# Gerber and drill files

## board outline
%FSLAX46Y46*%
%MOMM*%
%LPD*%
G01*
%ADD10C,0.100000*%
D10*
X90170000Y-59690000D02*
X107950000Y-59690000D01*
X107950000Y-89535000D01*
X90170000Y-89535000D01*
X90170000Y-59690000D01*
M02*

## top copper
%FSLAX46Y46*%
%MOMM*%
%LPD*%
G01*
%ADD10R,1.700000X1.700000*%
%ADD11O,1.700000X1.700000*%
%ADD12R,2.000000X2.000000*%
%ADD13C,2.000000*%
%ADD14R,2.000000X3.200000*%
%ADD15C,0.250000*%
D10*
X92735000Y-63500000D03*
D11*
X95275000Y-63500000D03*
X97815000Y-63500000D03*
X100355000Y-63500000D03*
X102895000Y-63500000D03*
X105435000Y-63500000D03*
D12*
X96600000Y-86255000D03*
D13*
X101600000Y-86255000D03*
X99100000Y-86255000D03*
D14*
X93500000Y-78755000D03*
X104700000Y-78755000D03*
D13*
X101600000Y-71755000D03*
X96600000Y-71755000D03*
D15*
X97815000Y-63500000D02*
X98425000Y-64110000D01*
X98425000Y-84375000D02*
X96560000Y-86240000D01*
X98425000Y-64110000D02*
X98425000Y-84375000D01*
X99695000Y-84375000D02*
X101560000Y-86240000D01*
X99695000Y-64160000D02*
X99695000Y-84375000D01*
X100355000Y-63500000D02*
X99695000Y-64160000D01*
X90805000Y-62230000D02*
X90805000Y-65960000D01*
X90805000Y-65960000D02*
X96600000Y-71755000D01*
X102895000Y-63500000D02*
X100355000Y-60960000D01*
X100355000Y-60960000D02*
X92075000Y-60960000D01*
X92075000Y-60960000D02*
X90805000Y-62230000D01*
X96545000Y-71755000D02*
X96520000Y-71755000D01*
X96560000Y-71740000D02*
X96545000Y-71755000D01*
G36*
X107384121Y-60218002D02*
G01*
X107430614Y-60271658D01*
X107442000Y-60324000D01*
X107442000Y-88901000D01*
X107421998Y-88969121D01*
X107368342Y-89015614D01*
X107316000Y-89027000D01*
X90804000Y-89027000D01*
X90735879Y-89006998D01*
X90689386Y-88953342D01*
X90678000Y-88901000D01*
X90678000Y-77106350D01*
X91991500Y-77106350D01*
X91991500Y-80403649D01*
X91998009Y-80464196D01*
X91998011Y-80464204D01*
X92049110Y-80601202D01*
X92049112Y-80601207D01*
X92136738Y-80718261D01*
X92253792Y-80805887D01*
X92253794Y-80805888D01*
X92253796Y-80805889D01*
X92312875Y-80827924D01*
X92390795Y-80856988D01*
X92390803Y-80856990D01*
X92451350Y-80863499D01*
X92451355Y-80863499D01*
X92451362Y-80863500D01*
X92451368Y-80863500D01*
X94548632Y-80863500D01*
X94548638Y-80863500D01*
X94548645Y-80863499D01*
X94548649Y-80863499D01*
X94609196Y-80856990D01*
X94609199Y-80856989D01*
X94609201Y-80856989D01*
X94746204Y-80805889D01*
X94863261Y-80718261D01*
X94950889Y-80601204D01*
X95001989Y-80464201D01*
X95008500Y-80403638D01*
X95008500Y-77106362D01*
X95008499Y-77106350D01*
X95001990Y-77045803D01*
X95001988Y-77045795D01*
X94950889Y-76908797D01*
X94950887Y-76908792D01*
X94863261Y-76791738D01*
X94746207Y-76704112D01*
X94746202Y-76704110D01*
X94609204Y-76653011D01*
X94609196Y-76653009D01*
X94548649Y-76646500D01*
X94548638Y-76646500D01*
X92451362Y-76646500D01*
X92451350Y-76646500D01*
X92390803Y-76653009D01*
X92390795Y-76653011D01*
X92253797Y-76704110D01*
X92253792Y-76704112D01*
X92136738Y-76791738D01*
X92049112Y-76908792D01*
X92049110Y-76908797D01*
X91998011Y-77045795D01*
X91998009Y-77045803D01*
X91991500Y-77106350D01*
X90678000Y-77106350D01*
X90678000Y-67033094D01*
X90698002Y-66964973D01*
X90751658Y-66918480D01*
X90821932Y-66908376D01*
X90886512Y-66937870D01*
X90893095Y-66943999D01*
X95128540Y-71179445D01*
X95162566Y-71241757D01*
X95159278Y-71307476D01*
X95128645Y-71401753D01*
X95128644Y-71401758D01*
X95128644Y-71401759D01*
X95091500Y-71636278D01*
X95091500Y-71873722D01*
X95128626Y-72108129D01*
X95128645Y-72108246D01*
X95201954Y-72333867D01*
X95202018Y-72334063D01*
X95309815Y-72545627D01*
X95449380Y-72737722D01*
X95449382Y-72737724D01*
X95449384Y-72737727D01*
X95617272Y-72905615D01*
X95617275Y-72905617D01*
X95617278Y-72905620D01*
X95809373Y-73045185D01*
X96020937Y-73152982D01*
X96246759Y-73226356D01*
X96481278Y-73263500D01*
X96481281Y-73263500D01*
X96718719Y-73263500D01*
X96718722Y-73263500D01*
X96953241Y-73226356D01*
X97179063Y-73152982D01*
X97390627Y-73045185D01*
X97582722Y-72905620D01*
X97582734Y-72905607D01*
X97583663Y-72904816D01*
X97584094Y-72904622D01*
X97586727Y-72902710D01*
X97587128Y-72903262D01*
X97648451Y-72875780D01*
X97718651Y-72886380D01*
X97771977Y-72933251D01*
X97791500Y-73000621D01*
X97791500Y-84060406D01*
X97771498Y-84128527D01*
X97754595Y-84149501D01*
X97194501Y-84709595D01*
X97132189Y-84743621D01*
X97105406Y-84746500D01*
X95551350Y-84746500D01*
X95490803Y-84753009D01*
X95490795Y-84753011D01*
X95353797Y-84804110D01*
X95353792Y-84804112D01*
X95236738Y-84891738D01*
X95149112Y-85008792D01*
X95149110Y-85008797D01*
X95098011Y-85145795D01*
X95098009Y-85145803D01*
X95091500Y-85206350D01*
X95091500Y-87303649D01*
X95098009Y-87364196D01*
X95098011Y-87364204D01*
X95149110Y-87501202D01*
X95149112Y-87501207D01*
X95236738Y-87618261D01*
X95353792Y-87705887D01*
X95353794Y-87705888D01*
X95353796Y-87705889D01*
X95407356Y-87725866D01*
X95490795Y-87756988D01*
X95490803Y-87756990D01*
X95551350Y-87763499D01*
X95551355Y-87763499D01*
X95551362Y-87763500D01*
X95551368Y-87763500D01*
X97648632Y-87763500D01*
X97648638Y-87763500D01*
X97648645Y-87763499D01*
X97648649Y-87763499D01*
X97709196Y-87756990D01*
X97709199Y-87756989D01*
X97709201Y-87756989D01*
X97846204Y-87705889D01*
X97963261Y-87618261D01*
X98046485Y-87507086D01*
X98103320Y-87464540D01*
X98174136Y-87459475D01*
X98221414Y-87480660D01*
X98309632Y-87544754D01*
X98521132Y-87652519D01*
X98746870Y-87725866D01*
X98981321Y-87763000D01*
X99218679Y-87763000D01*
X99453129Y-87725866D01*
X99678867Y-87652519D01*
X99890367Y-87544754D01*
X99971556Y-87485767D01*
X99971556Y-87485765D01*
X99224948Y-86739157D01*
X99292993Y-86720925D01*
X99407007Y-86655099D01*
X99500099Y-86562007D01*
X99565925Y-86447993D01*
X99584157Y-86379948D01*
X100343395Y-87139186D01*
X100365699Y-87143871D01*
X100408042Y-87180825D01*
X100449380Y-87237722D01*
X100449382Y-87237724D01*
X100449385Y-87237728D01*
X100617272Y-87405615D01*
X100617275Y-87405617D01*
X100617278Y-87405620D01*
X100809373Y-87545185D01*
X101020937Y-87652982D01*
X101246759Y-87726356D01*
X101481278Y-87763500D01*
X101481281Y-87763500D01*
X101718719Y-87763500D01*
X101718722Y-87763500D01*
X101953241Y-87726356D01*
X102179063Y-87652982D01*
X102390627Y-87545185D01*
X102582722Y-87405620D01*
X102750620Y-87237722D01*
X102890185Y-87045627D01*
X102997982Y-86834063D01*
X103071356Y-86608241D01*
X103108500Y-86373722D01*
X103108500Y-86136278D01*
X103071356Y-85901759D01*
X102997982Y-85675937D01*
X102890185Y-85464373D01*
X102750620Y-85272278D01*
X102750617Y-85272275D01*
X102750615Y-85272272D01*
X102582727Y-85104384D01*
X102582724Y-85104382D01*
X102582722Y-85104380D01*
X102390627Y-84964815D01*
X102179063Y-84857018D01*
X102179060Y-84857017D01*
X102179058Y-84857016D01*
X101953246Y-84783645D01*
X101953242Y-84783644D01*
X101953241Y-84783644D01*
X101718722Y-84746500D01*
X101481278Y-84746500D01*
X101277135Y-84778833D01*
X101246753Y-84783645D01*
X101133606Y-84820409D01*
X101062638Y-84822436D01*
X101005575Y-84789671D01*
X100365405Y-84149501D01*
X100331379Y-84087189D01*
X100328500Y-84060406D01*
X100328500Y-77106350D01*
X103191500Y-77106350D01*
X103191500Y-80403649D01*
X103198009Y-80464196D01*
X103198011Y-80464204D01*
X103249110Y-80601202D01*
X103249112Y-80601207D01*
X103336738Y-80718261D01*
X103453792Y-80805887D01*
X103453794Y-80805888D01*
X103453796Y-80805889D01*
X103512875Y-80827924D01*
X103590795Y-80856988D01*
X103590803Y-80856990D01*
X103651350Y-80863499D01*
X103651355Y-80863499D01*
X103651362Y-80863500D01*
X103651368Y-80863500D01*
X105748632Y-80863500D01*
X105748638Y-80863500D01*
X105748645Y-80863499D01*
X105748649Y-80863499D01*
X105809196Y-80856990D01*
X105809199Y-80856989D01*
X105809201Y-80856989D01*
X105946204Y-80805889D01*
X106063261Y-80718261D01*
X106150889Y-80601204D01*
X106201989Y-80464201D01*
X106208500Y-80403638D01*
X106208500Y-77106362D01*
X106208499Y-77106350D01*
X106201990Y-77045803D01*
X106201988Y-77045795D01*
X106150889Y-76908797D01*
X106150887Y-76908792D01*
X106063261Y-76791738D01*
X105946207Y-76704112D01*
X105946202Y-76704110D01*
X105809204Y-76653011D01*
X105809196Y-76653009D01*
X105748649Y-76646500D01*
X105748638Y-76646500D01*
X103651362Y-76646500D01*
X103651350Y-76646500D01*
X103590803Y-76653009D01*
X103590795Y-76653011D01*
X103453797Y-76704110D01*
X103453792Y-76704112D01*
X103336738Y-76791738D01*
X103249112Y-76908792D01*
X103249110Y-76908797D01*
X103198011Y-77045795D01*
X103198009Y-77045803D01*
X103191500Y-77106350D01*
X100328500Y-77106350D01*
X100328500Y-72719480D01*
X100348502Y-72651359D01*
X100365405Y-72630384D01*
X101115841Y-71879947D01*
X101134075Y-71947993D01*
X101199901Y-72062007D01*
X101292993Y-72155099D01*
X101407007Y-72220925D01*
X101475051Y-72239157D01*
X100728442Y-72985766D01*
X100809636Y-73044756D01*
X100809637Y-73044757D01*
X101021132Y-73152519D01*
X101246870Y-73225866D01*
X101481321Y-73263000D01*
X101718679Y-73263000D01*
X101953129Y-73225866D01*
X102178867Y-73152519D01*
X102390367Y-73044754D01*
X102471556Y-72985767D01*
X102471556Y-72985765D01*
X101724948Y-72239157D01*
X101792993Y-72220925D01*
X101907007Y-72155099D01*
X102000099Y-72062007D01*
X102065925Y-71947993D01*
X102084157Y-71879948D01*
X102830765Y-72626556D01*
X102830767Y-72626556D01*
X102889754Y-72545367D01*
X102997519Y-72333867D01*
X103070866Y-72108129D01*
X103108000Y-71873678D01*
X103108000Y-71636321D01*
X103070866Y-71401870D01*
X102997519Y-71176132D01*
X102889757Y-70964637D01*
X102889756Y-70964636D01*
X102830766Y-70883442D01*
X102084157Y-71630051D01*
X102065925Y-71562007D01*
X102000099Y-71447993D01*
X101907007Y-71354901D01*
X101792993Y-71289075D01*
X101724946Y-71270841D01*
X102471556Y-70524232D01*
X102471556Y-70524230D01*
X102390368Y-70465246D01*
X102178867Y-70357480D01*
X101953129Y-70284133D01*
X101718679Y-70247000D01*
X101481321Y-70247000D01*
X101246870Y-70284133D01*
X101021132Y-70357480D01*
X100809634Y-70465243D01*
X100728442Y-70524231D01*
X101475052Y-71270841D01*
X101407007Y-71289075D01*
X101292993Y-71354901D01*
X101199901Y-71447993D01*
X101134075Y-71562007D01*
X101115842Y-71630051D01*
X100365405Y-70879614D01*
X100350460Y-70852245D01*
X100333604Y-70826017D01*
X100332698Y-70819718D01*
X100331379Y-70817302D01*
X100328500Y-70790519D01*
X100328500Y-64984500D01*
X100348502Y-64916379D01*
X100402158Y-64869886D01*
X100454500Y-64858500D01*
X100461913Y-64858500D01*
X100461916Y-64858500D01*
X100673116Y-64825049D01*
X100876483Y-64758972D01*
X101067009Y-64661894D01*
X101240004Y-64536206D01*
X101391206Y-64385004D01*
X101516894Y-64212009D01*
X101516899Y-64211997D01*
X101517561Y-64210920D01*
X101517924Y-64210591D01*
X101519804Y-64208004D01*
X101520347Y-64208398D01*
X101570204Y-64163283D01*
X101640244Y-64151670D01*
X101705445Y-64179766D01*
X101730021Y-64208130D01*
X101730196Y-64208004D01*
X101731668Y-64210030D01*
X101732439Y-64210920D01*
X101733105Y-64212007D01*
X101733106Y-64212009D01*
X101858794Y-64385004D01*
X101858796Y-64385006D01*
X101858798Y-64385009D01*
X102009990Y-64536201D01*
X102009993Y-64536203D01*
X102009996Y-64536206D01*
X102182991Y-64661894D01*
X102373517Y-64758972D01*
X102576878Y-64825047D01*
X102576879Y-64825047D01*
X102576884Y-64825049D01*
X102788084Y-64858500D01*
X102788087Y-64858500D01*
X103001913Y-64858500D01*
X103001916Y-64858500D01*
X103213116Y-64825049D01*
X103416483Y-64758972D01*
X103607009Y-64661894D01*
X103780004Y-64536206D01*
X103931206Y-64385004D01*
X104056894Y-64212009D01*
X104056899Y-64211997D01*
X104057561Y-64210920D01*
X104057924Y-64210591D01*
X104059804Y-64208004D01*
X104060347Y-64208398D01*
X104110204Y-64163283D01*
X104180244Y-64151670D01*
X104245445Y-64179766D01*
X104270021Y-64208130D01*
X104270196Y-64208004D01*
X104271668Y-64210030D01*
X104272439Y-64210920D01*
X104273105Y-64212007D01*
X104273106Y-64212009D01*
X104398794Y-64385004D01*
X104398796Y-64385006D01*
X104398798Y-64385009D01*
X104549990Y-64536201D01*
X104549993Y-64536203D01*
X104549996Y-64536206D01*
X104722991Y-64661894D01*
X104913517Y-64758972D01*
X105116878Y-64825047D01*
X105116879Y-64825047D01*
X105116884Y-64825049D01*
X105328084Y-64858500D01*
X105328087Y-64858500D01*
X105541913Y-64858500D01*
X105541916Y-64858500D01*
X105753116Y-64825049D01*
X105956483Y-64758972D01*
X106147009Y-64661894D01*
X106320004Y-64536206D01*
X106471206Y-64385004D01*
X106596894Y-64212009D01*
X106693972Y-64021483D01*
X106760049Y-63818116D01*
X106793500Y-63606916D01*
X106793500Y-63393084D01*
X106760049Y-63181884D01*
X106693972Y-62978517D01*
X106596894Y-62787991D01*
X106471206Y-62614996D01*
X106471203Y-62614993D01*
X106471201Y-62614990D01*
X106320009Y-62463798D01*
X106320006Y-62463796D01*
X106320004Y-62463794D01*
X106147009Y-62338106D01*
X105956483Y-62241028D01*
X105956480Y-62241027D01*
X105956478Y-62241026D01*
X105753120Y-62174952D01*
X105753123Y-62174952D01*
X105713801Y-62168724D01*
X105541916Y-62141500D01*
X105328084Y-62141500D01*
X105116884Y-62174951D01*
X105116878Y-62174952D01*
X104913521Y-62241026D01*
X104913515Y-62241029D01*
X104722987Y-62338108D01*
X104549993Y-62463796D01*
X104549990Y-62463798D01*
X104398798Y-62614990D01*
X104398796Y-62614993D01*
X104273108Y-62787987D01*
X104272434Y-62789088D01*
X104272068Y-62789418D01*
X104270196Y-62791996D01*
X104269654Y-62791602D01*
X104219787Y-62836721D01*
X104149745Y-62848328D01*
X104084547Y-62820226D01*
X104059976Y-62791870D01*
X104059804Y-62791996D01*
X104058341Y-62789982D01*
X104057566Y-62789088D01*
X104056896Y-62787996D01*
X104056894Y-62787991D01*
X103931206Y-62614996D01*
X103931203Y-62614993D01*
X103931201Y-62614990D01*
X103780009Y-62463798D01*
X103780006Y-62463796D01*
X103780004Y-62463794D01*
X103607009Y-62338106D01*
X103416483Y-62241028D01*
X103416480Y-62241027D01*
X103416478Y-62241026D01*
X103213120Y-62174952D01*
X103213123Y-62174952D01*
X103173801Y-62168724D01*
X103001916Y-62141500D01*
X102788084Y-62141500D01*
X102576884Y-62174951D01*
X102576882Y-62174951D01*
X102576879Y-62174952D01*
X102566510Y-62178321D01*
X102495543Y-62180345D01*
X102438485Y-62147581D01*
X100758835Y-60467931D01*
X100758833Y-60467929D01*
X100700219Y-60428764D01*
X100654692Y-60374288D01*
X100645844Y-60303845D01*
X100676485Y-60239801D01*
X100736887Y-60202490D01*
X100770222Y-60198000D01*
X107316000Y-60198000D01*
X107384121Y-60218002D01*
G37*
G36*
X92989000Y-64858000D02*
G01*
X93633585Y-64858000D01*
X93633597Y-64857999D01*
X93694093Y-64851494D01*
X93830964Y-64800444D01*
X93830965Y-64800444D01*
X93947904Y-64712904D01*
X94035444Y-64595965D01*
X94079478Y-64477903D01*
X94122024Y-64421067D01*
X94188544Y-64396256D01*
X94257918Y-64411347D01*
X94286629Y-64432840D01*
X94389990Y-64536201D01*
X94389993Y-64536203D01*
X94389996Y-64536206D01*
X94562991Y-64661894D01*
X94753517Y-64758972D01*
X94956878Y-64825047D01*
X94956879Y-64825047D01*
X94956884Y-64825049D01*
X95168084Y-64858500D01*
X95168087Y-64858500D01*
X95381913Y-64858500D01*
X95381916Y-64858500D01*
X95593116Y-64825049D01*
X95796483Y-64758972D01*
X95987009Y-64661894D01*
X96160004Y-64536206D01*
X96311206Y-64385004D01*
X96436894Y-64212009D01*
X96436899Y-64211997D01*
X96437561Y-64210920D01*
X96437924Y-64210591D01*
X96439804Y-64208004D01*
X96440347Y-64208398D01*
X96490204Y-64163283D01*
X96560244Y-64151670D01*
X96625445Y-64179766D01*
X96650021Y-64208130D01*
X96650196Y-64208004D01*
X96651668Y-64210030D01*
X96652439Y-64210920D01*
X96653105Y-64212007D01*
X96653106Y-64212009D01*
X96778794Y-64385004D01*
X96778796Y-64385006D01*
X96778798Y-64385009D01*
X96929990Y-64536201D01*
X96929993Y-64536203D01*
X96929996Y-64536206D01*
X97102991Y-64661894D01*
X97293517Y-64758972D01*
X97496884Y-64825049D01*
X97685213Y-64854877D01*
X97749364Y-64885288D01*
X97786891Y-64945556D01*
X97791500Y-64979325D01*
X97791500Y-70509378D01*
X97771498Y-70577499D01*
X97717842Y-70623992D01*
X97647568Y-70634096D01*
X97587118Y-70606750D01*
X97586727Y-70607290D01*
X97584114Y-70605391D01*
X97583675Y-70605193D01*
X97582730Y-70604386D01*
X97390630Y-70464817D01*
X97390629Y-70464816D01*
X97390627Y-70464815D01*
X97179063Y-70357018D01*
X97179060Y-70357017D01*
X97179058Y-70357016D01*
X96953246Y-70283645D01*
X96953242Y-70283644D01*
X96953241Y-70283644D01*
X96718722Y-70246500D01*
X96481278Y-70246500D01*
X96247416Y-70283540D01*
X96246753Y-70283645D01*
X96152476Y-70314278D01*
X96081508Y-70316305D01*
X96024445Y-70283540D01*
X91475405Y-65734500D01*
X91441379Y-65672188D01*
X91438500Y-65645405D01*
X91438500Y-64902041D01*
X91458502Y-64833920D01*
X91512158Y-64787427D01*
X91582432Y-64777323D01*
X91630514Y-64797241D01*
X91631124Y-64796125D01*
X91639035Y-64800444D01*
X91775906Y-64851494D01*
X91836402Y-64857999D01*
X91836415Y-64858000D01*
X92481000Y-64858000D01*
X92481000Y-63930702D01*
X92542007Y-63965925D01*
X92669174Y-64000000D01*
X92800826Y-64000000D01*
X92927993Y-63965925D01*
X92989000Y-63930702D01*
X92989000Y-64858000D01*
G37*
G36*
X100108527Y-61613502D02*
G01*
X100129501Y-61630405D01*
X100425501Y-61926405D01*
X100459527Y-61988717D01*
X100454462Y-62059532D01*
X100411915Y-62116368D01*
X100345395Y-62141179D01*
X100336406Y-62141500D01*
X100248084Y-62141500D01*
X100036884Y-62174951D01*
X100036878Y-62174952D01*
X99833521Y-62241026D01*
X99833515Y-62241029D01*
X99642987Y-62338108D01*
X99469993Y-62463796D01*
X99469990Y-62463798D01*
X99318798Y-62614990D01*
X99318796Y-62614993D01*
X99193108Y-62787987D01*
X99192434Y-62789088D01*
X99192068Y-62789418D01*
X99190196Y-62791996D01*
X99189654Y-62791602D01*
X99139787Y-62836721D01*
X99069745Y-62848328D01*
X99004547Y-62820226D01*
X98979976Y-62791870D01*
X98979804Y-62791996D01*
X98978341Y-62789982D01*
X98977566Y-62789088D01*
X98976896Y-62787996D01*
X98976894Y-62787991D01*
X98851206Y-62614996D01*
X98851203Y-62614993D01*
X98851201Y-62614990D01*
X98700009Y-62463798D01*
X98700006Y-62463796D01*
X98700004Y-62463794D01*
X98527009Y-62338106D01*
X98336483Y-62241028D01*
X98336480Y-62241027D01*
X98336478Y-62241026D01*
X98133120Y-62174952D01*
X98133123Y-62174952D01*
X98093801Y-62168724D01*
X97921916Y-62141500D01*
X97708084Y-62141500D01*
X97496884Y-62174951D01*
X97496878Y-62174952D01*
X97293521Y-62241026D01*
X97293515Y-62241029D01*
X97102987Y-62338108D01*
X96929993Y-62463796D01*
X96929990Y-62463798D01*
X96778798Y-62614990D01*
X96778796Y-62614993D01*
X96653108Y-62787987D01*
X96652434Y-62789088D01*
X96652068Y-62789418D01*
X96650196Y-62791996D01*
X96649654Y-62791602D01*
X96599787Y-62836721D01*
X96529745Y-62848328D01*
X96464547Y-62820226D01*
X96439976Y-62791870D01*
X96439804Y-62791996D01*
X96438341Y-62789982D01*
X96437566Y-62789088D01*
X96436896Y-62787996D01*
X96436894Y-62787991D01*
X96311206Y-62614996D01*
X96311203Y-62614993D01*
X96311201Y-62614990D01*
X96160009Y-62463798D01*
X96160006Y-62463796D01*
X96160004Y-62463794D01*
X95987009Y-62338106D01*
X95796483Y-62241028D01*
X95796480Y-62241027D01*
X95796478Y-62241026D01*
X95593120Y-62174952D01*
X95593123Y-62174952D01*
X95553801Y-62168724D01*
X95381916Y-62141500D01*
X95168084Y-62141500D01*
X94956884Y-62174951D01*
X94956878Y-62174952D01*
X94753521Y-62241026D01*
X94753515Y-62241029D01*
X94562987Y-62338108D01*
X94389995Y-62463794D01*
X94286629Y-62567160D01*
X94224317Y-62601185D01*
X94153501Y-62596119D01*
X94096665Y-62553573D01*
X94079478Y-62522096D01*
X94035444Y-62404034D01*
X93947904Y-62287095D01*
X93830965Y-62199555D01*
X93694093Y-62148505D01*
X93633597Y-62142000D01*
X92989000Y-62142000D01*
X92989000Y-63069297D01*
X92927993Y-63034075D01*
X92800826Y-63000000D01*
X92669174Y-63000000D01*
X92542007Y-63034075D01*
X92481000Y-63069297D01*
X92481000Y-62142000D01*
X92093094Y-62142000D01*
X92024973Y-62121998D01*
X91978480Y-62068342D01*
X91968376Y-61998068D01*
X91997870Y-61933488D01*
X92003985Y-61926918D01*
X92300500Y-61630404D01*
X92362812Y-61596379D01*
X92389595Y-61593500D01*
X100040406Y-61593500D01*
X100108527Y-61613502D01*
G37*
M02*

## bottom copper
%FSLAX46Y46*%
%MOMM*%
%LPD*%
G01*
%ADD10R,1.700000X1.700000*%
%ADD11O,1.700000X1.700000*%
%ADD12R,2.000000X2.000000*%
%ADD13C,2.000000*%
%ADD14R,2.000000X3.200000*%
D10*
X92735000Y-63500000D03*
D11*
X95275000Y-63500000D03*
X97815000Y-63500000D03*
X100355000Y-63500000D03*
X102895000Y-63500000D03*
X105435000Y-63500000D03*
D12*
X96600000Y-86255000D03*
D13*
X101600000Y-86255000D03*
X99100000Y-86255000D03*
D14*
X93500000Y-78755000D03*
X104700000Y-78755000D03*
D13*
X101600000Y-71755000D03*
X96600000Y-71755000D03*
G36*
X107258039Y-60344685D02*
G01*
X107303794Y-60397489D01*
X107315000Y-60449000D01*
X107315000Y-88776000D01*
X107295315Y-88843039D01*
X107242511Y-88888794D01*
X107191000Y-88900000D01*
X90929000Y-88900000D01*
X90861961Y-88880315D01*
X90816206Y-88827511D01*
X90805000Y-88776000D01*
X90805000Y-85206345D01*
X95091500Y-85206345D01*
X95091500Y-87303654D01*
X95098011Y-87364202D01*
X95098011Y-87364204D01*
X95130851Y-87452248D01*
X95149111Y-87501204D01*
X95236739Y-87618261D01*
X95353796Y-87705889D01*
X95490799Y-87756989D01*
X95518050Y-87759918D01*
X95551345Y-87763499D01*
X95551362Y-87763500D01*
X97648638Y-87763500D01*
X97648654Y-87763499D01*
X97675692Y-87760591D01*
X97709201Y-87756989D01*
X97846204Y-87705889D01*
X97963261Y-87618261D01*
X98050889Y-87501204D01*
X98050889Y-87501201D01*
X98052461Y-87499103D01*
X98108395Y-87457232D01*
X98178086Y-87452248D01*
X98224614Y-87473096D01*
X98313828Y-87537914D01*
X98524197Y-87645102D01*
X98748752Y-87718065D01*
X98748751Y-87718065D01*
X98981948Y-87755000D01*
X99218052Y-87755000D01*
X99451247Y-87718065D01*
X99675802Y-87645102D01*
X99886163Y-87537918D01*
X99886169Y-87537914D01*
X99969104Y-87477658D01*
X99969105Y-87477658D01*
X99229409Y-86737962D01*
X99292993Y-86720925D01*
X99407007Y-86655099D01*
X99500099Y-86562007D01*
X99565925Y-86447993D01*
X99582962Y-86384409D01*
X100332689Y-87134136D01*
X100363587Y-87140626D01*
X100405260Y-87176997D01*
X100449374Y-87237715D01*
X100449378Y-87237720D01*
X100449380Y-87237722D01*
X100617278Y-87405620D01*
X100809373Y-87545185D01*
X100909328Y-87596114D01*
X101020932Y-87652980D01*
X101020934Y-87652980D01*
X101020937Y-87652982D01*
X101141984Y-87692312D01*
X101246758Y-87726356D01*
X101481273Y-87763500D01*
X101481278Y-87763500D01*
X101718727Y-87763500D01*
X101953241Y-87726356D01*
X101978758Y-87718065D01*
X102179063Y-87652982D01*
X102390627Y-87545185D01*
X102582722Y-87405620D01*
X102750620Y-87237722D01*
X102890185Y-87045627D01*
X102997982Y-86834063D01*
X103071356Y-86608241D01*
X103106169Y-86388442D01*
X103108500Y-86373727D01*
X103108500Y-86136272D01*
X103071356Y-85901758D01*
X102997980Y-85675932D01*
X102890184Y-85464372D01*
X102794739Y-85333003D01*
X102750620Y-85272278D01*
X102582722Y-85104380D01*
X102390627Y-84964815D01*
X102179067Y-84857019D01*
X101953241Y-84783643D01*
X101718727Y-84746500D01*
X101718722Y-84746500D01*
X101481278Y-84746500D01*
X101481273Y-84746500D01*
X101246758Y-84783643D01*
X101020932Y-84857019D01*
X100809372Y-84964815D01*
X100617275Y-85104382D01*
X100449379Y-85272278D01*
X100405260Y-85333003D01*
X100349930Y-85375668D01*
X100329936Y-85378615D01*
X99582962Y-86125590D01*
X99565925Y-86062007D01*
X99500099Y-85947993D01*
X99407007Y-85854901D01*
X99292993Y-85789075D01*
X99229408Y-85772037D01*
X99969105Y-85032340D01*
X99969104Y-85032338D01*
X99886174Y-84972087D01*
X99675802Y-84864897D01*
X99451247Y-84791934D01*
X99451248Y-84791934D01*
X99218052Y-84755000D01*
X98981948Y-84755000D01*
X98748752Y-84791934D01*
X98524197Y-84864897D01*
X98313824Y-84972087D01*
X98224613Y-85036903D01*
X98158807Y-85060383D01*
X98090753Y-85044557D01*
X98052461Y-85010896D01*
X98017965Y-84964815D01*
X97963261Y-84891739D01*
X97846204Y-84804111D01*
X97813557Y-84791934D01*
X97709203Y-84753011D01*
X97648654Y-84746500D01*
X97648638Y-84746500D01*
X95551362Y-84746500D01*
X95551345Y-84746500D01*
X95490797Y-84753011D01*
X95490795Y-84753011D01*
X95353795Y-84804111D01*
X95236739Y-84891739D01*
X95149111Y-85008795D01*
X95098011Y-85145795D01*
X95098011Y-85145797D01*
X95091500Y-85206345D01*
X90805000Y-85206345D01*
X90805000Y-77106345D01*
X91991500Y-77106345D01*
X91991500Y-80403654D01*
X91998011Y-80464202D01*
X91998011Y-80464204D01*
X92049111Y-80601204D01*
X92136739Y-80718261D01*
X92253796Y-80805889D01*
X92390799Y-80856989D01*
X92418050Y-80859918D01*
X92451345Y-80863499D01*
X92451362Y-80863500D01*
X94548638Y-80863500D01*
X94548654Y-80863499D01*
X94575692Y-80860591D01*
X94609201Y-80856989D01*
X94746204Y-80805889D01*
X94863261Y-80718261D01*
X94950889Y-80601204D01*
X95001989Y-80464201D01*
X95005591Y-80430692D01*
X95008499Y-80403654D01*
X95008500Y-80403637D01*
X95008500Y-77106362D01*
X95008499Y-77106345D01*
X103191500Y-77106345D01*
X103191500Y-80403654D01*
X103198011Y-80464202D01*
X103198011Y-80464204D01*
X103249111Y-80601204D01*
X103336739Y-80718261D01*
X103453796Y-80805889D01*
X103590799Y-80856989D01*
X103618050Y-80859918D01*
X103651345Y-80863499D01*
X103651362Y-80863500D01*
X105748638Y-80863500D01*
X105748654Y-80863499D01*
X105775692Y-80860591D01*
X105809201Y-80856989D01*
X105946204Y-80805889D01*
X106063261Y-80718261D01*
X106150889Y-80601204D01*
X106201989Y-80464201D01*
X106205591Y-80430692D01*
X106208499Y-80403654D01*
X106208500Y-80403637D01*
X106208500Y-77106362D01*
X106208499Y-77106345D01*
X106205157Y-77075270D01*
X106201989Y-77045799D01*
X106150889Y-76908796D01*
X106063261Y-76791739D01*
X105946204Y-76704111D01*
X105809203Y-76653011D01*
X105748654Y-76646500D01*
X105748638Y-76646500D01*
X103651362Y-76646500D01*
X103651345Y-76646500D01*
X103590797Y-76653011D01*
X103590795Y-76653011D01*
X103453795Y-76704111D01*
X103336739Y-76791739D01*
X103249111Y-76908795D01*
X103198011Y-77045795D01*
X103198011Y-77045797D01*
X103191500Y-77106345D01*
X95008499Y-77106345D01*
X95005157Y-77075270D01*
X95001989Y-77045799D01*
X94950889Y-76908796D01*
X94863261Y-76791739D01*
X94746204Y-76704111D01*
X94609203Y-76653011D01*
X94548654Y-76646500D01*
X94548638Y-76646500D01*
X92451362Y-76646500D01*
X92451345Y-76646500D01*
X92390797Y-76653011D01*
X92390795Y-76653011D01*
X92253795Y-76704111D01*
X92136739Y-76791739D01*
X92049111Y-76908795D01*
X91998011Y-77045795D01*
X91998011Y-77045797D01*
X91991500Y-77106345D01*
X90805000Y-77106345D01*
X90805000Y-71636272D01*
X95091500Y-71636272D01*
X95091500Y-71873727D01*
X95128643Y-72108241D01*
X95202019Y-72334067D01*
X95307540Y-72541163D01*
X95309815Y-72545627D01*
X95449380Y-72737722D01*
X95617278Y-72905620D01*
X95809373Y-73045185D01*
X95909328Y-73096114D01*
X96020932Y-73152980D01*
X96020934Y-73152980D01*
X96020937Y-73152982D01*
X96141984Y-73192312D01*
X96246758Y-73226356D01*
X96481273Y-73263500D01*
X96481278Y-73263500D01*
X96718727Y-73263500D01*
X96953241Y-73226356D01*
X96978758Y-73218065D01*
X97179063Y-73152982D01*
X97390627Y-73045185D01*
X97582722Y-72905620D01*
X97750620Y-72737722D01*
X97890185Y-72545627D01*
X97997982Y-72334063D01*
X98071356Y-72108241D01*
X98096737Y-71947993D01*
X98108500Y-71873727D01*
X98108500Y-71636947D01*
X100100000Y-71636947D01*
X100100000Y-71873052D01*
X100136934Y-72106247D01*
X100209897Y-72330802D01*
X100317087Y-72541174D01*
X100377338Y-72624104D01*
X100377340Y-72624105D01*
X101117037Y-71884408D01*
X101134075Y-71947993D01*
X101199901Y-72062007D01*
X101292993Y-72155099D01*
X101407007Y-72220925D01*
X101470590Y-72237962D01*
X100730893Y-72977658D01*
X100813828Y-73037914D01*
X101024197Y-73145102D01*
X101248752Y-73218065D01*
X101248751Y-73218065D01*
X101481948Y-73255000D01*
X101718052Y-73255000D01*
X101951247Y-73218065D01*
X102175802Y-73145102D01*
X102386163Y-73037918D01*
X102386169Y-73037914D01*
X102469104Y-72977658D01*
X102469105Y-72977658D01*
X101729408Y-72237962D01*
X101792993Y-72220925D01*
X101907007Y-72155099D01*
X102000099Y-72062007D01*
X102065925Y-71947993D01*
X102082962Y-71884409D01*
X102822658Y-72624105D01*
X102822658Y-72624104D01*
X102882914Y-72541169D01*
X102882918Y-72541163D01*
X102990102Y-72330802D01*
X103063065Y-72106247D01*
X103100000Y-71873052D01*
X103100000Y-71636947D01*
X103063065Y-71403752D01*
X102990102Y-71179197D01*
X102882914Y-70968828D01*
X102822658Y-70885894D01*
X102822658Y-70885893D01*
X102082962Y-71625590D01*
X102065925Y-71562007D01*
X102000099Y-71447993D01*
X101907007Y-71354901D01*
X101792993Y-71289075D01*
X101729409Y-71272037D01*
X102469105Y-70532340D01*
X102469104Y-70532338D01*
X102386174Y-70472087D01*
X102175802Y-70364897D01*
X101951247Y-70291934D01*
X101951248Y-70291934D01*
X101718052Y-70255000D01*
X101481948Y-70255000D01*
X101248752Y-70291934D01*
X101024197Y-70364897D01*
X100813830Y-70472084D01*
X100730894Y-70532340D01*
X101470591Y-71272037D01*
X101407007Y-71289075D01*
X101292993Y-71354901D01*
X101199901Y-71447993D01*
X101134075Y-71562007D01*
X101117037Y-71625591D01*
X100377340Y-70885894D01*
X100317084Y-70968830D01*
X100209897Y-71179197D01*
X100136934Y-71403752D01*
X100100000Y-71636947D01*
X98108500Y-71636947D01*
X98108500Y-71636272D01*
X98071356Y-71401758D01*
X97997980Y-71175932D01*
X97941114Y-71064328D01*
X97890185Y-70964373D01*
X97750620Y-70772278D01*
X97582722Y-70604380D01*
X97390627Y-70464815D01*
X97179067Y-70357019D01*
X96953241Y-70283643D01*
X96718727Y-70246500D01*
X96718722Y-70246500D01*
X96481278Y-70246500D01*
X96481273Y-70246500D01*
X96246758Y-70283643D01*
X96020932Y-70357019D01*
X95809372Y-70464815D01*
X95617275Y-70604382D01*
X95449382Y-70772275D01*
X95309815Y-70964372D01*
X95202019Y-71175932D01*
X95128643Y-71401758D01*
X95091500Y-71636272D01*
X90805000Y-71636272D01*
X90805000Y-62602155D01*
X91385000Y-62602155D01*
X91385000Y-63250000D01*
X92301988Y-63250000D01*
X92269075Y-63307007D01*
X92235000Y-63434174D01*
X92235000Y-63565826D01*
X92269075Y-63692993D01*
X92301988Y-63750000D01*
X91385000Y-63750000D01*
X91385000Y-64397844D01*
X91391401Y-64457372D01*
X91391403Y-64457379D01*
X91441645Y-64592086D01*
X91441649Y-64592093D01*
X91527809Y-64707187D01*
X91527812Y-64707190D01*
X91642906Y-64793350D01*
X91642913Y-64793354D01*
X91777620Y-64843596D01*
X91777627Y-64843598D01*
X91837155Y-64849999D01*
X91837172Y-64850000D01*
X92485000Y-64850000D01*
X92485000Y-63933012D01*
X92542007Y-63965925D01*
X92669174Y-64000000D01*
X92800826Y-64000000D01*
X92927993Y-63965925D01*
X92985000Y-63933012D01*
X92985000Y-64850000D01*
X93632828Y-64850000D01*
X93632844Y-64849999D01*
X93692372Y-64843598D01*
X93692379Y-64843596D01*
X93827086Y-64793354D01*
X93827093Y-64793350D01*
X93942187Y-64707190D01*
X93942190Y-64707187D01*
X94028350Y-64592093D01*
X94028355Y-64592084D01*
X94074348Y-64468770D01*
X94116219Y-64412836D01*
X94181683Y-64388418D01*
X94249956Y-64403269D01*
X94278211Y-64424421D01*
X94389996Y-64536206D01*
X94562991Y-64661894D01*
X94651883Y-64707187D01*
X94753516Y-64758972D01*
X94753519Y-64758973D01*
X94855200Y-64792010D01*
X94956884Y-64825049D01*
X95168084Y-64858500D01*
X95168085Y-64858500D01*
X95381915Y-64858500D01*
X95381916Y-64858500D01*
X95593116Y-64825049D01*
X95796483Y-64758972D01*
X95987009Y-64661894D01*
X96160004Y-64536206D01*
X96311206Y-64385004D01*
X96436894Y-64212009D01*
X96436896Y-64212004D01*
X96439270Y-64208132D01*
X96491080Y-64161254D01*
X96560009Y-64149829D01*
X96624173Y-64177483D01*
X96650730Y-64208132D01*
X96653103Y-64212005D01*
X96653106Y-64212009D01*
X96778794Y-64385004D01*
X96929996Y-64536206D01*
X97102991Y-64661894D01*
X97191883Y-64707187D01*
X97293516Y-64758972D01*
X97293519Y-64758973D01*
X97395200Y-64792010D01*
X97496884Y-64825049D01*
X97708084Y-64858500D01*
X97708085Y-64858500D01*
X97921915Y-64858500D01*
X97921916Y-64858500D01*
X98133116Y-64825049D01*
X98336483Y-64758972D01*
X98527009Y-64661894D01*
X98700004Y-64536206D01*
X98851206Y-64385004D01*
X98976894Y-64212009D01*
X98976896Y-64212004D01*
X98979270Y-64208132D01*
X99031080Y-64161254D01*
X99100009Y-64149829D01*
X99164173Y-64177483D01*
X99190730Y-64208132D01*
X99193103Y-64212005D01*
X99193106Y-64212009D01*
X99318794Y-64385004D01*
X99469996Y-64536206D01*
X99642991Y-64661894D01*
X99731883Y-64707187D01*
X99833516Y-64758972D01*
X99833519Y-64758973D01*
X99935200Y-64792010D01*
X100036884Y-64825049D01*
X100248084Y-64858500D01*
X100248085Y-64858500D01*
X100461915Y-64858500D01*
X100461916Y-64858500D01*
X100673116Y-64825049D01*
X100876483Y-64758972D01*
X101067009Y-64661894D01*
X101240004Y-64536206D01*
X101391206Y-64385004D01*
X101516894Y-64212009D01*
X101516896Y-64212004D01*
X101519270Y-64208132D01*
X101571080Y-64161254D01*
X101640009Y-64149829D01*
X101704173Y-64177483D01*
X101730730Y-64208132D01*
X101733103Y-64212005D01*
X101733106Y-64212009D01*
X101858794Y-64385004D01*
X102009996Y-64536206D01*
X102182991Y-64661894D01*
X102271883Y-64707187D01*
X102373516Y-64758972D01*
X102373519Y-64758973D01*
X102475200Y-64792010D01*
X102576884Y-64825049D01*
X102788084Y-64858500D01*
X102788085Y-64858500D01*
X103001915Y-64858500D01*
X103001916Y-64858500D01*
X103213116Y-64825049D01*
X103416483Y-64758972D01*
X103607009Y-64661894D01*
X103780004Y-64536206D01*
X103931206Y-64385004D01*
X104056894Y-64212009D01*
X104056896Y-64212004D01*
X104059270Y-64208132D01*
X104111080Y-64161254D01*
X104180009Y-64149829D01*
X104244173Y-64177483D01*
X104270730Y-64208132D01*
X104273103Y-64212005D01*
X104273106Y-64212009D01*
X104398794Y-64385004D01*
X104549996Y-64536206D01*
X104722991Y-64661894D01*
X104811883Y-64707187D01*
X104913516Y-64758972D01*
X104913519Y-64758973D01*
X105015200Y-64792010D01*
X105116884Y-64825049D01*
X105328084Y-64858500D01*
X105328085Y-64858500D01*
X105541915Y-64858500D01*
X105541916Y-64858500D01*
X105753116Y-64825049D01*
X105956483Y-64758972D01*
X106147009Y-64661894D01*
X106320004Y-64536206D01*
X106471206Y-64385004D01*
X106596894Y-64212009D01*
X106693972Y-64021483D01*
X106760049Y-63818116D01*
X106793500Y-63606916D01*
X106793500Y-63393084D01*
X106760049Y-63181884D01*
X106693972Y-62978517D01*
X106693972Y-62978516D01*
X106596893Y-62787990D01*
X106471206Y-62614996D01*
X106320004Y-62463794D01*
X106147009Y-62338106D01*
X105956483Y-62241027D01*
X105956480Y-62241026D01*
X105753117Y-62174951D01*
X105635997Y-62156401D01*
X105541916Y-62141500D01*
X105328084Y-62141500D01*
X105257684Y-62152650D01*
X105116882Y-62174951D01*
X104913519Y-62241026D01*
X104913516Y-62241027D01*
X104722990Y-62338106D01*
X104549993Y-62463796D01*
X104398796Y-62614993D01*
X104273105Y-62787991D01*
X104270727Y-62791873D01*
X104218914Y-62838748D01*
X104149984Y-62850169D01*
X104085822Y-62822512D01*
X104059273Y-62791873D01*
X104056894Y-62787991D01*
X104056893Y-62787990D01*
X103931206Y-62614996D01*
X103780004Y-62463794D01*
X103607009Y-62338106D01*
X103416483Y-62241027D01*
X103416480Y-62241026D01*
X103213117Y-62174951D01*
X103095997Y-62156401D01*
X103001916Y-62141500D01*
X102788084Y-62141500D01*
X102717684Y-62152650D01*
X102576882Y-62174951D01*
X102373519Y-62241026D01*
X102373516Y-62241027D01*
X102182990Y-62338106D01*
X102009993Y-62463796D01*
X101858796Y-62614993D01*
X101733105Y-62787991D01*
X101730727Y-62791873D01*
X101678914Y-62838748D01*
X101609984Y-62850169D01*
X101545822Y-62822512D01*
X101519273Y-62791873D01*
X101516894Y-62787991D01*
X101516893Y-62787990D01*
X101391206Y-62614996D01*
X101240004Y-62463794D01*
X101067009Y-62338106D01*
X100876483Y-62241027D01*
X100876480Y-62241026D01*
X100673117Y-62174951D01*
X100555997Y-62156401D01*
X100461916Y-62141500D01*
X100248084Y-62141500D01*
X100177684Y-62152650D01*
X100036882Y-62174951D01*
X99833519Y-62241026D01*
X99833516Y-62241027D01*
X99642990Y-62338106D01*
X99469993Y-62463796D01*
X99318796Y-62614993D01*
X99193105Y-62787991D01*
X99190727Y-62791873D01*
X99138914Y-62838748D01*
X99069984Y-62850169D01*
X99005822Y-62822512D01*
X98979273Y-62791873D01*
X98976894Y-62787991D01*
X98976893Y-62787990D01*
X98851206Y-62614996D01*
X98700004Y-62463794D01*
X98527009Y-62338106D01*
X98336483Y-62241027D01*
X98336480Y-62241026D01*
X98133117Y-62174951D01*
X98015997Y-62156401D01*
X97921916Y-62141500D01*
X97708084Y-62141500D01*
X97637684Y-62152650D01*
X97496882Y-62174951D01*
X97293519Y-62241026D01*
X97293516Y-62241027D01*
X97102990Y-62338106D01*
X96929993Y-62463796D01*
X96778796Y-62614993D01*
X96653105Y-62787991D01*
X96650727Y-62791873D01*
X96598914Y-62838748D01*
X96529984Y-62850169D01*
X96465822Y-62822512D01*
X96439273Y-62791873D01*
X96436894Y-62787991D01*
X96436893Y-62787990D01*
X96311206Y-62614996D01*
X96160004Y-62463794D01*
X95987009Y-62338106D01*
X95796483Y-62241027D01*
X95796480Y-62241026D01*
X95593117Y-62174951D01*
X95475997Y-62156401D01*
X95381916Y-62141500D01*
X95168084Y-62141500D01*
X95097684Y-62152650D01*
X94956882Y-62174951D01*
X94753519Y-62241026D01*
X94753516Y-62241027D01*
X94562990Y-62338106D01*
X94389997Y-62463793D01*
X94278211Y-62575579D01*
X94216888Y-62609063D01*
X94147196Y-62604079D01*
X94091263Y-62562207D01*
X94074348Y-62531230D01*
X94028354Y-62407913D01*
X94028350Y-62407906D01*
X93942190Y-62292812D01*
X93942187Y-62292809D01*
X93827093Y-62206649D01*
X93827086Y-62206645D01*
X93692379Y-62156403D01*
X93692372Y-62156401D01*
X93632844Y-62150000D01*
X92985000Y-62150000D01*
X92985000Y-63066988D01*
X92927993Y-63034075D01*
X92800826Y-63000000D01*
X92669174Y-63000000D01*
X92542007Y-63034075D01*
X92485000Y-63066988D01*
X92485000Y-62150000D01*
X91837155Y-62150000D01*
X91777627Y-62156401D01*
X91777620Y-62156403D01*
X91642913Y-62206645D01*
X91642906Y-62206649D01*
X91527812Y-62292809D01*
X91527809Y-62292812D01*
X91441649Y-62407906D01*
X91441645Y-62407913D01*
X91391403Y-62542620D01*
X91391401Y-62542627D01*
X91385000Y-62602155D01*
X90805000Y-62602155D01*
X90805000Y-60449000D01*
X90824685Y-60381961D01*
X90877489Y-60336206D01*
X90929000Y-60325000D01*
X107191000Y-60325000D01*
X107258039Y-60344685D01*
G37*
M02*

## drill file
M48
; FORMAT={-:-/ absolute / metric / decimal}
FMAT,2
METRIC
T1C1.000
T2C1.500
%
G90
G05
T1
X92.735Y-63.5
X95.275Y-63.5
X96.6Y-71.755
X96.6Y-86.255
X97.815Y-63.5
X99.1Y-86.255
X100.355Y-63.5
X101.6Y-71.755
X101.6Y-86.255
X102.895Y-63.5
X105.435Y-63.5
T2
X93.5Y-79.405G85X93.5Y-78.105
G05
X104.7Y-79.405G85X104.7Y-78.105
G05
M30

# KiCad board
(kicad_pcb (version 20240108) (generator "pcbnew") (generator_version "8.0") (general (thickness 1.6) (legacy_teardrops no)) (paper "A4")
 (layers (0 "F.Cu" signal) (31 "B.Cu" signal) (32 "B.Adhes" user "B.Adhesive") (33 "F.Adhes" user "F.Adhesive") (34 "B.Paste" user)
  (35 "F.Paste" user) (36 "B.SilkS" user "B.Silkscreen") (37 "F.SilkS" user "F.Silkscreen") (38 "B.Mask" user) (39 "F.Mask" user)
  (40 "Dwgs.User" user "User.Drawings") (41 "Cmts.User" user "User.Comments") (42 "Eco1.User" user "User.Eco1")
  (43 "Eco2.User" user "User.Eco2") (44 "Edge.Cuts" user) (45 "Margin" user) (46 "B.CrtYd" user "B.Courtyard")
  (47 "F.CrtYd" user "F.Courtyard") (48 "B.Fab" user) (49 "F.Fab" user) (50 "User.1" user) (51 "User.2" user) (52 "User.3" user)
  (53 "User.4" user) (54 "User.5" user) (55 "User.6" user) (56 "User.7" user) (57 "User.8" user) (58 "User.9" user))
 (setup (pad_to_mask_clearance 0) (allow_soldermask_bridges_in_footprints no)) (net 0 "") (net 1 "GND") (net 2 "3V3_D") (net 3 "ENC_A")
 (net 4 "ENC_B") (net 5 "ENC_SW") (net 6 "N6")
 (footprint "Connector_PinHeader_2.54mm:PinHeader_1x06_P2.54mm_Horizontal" (layer "F.Cu") (at 92.735 63.5 90)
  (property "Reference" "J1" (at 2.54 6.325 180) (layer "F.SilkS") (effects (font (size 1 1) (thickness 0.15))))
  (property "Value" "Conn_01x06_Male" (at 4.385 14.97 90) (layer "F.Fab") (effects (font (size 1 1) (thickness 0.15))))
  (pad "1" thru_hole rect (at 0 0 90) (size 1.7 1.7) (drill 1) (layers "*.Cu" "*.Mask") (remove_unused_layers no) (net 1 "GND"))
  (pad "2" thru_hole oval (at 0 2.54 90) (size 1.7 1.7) (drill 1) (layers "*.Cu" "*.Mask") (remove_unused_layers no) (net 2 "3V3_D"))
  (pad "3" thru_hole oval (at 0 5.08 90) (size 1.7 1.7) (drill 1) (layers "*.Cu" "*.Mask") (remove_unused_layers no) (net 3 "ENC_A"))
  (pad "4" thru_hole oval (at 0 7.62 90) (size 1.7 1.7) (drill 1) (layers "*.Cu" "*.Mask") (remove_unused_layers no) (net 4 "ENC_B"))
  (pad "5" thru_hole oval (at 0 10.16 90) (size 1.7 1.7) (drill 1) (layers "*.Cu" "*.Mask") (remove_unused_layers no) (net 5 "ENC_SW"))
  (pad "6" thru_hole oval (at 0 12.7 90) (size 1.7 1.7) (drill 1) (layers "*.Cu" "*.Mask") (remove_unused_layers no) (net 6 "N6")))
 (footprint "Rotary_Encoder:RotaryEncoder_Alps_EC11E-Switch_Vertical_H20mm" (layer "F.Cu") (at 96.6 86.255 90)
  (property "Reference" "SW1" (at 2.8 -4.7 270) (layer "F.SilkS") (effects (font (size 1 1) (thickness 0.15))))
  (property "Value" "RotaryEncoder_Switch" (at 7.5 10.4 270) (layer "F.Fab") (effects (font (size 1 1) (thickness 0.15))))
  (pad "A" thru_hole rect (at 0 0 90) (size 2 2) (drill 1) (layers "*.Cu" "*.Mask") (remove_unused_layers no) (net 3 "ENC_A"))
  (pad "B" thru_hole circle (at 0 5 90) (size 2 2) (drill 1) (layers "*.Cu" "*.Mask") (remove_unused_layers no) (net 4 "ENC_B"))
  (pad "C" thru_hole circle (at 0 2.5 90) (size 2 2) (drill 1) (layers "*.Cu" "*.Mask") (remove_unused_layers no) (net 1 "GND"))
  (pad "MP" thru_hole rect (at 7.5 -3.1 90) (size 3.2 2) (drill oval 2.8 1.5) (layers "*.Cu" "*.Mask") (remove_unused_layers no))
  (pad "MP" thru_hole rect (at 7.5 8.1 90) (size 3.2 2) (drill oval 2.8 1.5) (layers "*.Cu" "*.Mask") (remove_unused_layers no))
  (pad "S1" thru_hole circle (at 14.5 5 90) (size 2 2) (drill 1) (layers "*.Cu" "*.Mask") (remove_unused_layers no) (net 1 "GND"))
  (pad "S2" thru_hole circle (at 14.5 0 90) (size 2 2) (drill 1) (layers "*.Cu" "*.Mask") (remove_unused_layers no) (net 5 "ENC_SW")))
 (gr_rect (start 90.17 59.69) (end 107.95 89.535) (stroke (width 0.1) (type solid)) (fill none) (layer "Edge.Cuts"))
 (segment (start 97.815 63.5) (end 98.425 64.11) (width 0.25) (layer "F.Cu") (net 3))
 (segment (start 98.425 84.375) (end 96.56 86.24) (width 0.25) (layer "F.Cu") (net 3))
 (segment (start 98.425 64.11) (end 98.425 84.375) (width 0.25) (layer "F.Cu") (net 3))
 (segment (start 99.695 84.375) (end 101.56 86.24) (width 0.25) (layer "F.Cu") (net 4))
 (segment (start 99.695 64.16) (end 99.695 84.375) (width 0.25) (layer "F.Cu") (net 4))
 (segment (start 100.355 63.5) (end 99.695 64.16) (width 0.25) (layer "F.Cu") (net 4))
 (segment (start 90.805 62.23) (end 90.805 65.96) (width 0.25) (layer "F.Cu") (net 5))
 (segment (start 90.805 65.96) (end 96.6 71.755) (width 0.25) (layer "F.Cu") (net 5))
 (segment (start 102.895 63.5) (end 100.355 60.96) (width 0.25) (layer "F.Cu") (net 5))
 (segment (start 100.355 60.96) (end 92.075 60.96) (width 0.25) (layer "F.Cu") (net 5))
 (segment (start 92.075 60.96) (end 90.805 62.23) (width 0.25) (layer "F.Cu") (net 5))
 (segment (start 96.545 71.755) (end 96.52 71.755) (width 0.25) (layer "F.Cu") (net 5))
 (segment (start 96.56 71.74) (end 96.545 71.755) (width 0.25) (layer "F.Cu") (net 5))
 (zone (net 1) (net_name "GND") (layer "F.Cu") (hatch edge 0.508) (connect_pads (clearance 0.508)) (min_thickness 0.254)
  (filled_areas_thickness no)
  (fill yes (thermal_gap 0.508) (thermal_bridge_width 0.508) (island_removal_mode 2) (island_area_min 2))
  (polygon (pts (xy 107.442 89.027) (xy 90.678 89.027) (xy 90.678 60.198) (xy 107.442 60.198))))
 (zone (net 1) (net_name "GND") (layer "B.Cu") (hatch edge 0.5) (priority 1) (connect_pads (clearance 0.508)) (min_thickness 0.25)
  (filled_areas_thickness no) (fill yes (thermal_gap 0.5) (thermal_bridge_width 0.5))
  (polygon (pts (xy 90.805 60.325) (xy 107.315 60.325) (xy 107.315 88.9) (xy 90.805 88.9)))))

